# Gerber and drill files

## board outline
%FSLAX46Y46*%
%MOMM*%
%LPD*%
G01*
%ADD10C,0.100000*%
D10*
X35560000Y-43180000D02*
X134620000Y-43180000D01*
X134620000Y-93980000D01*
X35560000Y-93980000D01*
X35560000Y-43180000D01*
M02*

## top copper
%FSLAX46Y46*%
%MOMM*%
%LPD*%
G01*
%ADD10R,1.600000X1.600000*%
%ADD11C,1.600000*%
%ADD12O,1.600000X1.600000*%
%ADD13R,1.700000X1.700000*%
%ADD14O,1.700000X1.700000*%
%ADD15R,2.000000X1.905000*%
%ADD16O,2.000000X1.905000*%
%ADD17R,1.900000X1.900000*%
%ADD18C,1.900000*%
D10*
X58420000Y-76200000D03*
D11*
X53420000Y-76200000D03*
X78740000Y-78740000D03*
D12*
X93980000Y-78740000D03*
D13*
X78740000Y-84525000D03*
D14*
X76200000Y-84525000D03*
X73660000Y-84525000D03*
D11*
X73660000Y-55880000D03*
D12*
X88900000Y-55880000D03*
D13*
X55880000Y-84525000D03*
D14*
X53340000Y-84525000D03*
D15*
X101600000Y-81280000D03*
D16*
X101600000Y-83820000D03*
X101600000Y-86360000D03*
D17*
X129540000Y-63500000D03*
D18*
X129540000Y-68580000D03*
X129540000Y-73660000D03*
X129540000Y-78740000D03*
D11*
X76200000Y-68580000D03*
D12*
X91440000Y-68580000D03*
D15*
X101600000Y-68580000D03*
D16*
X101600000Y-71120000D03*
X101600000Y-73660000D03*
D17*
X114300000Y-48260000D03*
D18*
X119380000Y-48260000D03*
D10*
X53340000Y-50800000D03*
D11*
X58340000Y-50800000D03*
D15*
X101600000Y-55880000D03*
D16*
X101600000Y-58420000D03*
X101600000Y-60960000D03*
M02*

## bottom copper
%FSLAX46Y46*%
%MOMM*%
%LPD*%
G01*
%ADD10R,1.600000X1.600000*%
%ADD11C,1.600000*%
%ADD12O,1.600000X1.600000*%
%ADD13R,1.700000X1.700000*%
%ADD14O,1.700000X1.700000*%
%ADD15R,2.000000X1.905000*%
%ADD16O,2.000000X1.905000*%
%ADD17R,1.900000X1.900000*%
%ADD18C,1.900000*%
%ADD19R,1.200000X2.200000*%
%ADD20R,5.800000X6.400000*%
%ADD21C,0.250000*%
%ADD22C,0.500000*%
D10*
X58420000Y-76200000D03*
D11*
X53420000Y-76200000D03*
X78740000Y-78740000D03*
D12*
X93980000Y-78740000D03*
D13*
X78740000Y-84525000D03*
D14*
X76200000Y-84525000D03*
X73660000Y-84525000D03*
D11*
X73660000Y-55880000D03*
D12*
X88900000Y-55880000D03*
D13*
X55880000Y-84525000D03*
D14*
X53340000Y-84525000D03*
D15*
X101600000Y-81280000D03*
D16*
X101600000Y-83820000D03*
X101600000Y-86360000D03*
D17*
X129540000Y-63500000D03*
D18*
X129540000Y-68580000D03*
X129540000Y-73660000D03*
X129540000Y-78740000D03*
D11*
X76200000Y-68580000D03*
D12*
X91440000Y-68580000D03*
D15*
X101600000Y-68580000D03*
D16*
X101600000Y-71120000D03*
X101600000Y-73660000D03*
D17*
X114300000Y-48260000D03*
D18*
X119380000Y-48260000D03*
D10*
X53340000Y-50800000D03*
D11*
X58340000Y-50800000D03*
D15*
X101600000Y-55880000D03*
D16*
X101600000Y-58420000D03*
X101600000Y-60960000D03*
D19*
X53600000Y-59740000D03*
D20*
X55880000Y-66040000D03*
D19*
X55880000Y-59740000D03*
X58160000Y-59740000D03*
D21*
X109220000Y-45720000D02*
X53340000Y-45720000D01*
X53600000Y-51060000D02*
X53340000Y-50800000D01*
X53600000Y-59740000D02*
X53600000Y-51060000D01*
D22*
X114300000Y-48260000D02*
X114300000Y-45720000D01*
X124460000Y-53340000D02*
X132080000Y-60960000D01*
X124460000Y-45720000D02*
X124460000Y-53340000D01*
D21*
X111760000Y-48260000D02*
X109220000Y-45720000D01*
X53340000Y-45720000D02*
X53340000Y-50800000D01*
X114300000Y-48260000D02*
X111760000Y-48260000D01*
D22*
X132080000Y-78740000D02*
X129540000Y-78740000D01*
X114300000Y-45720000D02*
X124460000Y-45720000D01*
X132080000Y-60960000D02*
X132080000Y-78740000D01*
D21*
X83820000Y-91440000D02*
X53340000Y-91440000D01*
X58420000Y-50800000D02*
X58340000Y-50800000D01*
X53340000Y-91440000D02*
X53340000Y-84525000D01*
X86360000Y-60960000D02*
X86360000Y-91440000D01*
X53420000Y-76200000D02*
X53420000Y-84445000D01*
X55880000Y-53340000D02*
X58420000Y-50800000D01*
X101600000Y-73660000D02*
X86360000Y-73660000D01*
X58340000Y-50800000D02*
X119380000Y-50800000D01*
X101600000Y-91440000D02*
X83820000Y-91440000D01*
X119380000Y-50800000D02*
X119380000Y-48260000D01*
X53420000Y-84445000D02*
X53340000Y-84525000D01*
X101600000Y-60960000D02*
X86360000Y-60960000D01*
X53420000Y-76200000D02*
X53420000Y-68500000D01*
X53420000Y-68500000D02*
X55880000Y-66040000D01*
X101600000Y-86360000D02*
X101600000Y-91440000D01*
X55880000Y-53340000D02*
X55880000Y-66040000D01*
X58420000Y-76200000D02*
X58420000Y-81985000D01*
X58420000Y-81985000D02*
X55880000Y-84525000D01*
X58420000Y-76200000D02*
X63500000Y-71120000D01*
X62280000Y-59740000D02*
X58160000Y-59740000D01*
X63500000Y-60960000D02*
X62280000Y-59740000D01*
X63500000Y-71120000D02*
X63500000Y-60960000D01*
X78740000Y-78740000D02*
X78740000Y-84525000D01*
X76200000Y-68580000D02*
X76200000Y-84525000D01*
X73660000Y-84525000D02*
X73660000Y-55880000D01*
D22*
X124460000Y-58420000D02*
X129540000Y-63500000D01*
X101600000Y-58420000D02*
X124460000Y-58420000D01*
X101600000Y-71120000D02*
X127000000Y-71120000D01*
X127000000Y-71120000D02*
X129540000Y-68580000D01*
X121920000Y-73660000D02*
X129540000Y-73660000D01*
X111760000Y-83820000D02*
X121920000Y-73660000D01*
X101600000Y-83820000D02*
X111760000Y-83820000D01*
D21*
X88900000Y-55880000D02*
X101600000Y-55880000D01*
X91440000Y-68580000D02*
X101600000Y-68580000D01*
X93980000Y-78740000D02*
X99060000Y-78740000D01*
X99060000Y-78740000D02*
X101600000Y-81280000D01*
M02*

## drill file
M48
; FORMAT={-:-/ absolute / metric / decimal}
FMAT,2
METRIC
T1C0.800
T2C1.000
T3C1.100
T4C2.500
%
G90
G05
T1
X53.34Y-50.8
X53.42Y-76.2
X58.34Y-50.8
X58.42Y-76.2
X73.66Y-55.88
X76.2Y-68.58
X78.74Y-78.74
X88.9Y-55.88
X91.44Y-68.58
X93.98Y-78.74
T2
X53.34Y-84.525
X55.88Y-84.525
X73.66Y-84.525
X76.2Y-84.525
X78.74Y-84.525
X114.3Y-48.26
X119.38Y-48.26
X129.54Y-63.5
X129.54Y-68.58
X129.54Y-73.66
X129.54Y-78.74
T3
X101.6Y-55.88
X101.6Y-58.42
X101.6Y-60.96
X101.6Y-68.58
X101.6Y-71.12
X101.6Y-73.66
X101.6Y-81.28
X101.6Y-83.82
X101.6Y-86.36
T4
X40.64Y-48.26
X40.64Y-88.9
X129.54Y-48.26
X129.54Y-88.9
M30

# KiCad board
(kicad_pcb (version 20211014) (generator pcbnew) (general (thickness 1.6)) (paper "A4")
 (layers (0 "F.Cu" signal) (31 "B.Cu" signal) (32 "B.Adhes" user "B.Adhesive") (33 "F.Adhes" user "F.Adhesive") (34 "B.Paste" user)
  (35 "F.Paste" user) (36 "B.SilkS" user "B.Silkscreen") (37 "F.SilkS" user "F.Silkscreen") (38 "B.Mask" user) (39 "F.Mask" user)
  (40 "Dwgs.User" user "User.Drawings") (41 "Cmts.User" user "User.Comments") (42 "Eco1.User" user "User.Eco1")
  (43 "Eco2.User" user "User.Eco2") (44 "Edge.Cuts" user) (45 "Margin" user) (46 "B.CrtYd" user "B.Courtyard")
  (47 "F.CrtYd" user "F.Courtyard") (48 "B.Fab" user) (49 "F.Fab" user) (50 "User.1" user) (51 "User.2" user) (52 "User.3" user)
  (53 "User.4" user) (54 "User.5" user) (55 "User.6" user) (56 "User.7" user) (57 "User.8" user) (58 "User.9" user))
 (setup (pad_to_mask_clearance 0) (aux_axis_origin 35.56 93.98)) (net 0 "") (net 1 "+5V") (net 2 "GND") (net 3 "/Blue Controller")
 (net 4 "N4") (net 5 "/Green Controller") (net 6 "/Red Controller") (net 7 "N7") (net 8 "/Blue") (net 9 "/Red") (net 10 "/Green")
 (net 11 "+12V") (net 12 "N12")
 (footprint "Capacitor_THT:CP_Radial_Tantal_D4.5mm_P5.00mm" (layer "F.Cu") (at 58.42 76.2 180)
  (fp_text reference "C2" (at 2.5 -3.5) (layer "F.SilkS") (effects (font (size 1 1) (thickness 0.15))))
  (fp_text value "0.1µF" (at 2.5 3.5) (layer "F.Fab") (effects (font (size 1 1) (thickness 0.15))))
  (pad "1" thru_hole rect (at 0 0 180) (size 1.6 1.6) (drill 0.8) (layers *.Cu *.Mask) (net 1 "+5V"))
  (pad "2" thru_hole circle (at 5 0 180) (size 1.6 1.6) (drill 0.8) (layers *.Cu *.Mask) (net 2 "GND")))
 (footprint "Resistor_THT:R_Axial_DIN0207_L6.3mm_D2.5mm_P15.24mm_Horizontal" (layer "F.Cu") (at 78.74 78.74)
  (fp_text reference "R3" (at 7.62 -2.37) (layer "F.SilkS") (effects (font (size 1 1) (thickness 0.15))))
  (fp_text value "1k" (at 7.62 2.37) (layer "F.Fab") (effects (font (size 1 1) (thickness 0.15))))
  (pad "1" thru_hole circle (at 0 0) (size 1.6 1.6) (drill 0.8) (layers *.Cu *.Mask) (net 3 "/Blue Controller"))
  (pad "2" thru_hole oval (at 15.24 0) (size 1.6 1.6) (drill 0.8) (layers *.Cu *.Mask) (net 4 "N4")))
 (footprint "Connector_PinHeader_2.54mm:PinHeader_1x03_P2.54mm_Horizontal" (layer "F.Cu") (at 78.74 84.525 -90)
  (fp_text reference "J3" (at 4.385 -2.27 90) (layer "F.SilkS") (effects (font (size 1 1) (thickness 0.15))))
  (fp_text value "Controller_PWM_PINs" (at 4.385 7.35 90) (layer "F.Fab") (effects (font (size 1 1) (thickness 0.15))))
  (pad "1" thru_hole rect (at 0 0 270) (size 1.7 1.7) (drill 1) (layers *.Cu *.Mask) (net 3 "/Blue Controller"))
  (pad "2" thru_hole oval (at 0 2.54 270) (size 1.7 1.7) (drill 1) (layers *.Cu *.Mask) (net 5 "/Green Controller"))
  (pad "3" thru_hole oval (at 0 5.08 270) (size 1.7 1.7) (drill 1) (layers *.Cu *.Mask) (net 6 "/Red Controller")))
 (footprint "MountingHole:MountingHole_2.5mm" (layer "F.Cu") (at 129.54 48.26)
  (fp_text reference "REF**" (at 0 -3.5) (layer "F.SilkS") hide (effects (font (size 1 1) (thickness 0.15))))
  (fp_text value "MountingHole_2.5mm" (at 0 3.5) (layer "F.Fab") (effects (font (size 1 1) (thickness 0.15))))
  (pad "" np_thru_hole circle (at 0 0) (size 2.5 2.5) (drill 2.5) (layers *.Cu *.Mask)))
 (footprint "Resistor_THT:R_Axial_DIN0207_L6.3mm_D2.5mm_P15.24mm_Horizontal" (layer "F.Cu") (at 73.66 55.88)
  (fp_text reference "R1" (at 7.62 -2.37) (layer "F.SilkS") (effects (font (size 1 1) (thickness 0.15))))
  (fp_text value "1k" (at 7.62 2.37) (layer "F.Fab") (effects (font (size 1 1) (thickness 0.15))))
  (pad "1" thru_hole circle (at 0 0) (size 1.6 1.6) (drill 0.8) (layers *.Cu *.Mask) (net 6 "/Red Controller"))
  (pad "2" thru_hole oval (at 15.24 0) (size 1.6 1.6) (drill 0.8) (layers *.Cu *.Mask) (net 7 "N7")))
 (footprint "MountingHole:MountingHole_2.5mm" (layer "F.Cu") (at 40.64 48.26)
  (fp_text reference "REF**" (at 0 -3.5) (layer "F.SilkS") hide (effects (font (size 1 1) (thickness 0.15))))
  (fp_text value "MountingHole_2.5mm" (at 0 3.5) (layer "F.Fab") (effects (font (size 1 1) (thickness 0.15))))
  (pad "" np_thru_hole circle (at 0 0) (size 2.5 2.5) (drill 2.5) (layers *.Mask)))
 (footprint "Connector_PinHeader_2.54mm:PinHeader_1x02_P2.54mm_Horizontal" (layer "F.Cu") (at 55.88 84.525 -90)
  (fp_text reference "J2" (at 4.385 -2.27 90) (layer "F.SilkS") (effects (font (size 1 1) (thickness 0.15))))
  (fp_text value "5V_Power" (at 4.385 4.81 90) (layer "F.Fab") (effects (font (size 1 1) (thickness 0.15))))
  (pad "1" thru_hole rect (at 0 0 270) (size 1.7 1.7) (drill 1) (layers *.Cu *.Mask) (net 1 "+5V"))
  (pad "2" thru_hole oval (at 0 2.54 270) (size 1.7 1.7) (drill 1) (layers *.Cu *.Mask) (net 2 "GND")))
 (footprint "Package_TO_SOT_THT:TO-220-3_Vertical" (layer "F.Cu") (at 101.6 81.28 -90)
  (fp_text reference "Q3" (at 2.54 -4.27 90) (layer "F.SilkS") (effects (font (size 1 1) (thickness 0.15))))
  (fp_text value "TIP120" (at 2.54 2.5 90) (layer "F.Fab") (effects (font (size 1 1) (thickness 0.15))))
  (pad "1" thru_hole rect (at 0 0 270) (size 1.905 2) (drill 1.1) (layers *.Cu *.Mask) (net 4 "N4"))
  (pad "2" thru_hole oval (at 2.54 0 270) (size 1.905 2) (drill 1.1) (layers *.Cu *.Mask) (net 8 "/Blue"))
  (pad "3" thru_hole oval (at 5.08 0 270) (size 1.905 2) (drill 1.1) (layers *.Cu *.Mask) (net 2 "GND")))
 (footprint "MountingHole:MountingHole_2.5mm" (layer "F.Cu") (at 129.54 88.9)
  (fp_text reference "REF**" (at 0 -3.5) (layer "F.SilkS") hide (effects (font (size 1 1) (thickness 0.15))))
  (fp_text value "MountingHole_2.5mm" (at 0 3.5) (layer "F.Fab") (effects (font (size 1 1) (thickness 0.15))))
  (pad "" np_thru_hole circle (at 0 0) (size 2.5 2.5) (drill 2.5) (layers *.Cu *.Mask)))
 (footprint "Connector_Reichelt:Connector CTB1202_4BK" (layer "F.Cu") (at 129.54 63.5 -90)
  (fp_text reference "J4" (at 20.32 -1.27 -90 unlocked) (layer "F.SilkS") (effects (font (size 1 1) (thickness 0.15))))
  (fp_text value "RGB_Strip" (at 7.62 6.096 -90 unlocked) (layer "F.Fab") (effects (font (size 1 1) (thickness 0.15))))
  (pad "1" thru_hole rect (at 0 0 270) (size 1.9 1.9) (drill 1) (layers *.Cu *.Mask) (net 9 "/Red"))
  (pad "2" thru_hole circle (at 5.08 0 270) (size 1.9 1.9) (drill 1) (layers *.Cu *.Mask) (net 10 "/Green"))
  (pad "3" thru_hole circle (at 10.16 0 270) (size 1.9 1.9) (drill 1) (layers *.Cu *.Mask) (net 8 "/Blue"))
  (pad "4" thru_hole circle (at 15.24 0 270) (size 1.9 1.9) (drill 1) (layers *.Cu *.Mask) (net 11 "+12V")))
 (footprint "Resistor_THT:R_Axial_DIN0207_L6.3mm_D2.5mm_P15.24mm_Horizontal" (layer "F.Cu") (at 76.2 68.58)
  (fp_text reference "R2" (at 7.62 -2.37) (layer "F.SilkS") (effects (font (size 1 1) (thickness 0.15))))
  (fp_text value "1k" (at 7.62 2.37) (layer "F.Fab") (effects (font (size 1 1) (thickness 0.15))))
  (pad "1" thru_hole circle (at 0 0) (size 1.6 1.6) (drill 0.8) (layers *.Cu *.Mask) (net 5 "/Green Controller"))
  (pad "2" thru_hole oval (at 15.24 0) (size 1.6 1.6) (drill 0.8) (layers *.Cu *.Mask) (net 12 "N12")))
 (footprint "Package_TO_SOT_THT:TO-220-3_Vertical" (layer "F.Cu") (at 101.6 68.58 -90)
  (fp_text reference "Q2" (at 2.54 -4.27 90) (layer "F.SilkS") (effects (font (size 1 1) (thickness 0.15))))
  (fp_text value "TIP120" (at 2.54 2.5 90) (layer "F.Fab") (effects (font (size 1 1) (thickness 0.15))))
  (pad "1" thru_hole rect (at 0 0 270) (size 1.905 2) (drill 1.1) (layers *.Cu *.Mask) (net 12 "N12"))
  (pad "2" thru_hole oval (at 2.54 0 270) (size 1.905 2) (drill 1.1) (layers *.Cu *.Mask) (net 10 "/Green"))
  (pad "3" thru_hole oval (at 5.08 0 270) (size 1.905 2) (drill 1.1) (layers *.Cu *.Mask) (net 2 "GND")))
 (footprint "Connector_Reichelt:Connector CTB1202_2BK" (layer "F.Cu") (at 114.3 48.26)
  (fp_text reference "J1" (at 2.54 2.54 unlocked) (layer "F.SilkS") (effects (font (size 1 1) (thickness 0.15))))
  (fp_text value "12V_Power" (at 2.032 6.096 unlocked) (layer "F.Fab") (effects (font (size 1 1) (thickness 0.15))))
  (pad "1" thru_hole rect (at 0 0) (size 1.9 1.9) (drill 1) (layers *.Cu *.Mask) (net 11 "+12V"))
  (pad "2" thru_hole circle (at 5.08 0) (size 1.9 1.9) (drill 1) (layers *.Cu *.Mask) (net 2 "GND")))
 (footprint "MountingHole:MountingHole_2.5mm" (layer "F.Cu") (at 40.64 88.9)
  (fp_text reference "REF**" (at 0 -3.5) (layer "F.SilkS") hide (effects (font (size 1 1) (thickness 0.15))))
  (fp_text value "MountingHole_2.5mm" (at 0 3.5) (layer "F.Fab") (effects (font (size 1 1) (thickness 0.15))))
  (pad "" np_thru_hole circle (at 0 0) (size 2.5 2.5) (drill 2.5) (layers *.Cu *.Mask)))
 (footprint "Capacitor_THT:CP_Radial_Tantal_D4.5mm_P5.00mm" (layer "F.Cu") (at 53.34 50.8)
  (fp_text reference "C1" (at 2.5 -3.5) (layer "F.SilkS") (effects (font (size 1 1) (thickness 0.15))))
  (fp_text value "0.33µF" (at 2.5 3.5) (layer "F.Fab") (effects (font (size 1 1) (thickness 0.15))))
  (pad "1" thru_hole rect (at 0 0) (size 1.6 1.6) (drill 0.8) (layers *.Cu *.Mask) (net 11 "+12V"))
  (pad "2" thru_hole circle (at 5 0) (size 1.6 1.6) (drill 0.8) (layers *.Cu *.Mask) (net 2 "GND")))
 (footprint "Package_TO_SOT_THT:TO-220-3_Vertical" (layer "F.Cu") (at 101.6 55.88 -90)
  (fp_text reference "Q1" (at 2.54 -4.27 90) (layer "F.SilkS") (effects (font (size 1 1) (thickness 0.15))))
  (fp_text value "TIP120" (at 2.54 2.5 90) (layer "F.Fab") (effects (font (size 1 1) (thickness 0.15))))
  (pad "1" thru_hole rect (at 0 0 270) (size 1.905 2) (drill 1.1) (layers *.Cu *.Mask) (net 7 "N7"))
  (pad "2" thru_hole oval (at 2.54 0 270) (size 1.905 2) (drill 1.1) (layers *.Cu *.Mask) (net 9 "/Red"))
  (pad "3" thru_hole oval (at 5.08 0 270) (size 1.905 2) (drill 1.1) (layers *.Cu *.Mask) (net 2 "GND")))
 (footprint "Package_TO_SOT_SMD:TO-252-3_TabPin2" (layer "B.Cu") (at 55.88 63.94 -90)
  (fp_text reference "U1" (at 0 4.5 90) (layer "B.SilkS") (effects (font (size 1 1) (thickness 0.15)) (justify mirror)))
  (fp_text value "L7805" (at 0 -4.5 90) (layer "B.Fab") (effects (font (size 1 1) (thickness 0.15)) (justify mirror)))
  (pad "" smd rect (at 0.425 1.525 270) (size 3.05 2.75) (layers "B.Paste"))
  (pad "" smd rect (at 0.425 -1.525 270) (size 3.05 2.75) (layers "B.Paste"))
  (pad "" smd rect (at 3.775 -1.525 270) (size 3.05 2.75) (layers "B.Paste"))
  (pad "" smd rect (at 3.775 1.525 270) (size 3.05 2.75) (layers "B.Paste"))
  (pad "1" smd rect (at -4.2 2.28 270) (size 2.2 1.2) (layers "B.Cu" "B.Paste" "B.Mask") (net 11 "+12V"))
  (pad "2" smd rect (at 2.1 0 270) (size 6.4 5.8) (layers "B.Cu" "B.Mask") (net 2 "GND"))
  (pad "2" smd rect (at -4.2 0 270) (size 2.2 1.2) (layers "B.Cu" "B.Paste" "B.Mask") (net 2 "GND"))
  (pad "3" smd rect (at -4.2 -2.28 270) (size 2.2 1.2) (layers "B.Cu" "B.Paste" "B.Mask") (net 1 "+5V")))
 (gr_rect (start 35.56 43.18) (end 134.62 93.98) (layer "Edge.Cuts") (width 0.1) (fill none))
 (segment (start 109.22 45.72) (end 53.34 45.72) (width 0.25) (layer "B.Cu") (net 11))
 (segment (start 53.6 51.06) (end 53.34 50.8) (width 0.25) (layer "B.Cu") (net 11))
 (segment (start 53.6 59.74) (end 53.6 51.06) (width 0.25) (layer "B.Cu") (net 11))
 (segment (start 114.3 48.26) (end 114.3 45.72) (width 0.5) (layer "B.Cu") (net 11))
 (segment (start 124.46 53.34) (end 132.08 60.96) (width 0.5) (layer "B.Cu") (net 11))
 (segment (start 124.46 45.72) (end 124.46 53.34) (width 0.5) (layer "B.Cu") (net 11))
 (segment (start 111.76 48.26) (end 109.22 45.72) (width 0.25) (layer "B.Cu") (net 11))
 (segment (start 53.34 45.72) (end 53.34 50.8) (width 0.25) (layer "B.Cu") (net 11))
 (segment (start 114.3 48.26) (end 111.76 48.26) (width 0.25) (layer "B.Cu") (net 11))
 (segment (start 132.08 78.74) (end 129.54 78.74) (width 0.5) (layer "B.Cu") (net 11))
 (segment (start 114.3 45.72) (end 124.46 45.72) (width 0.5) (layer "B.Cu") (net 11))
 (segment (start 132.08 60.96) (end 132.08 78.74) (width 0.5) (layer "B.Cu") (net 11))
 (segment (start 83.82 91.44) (end 53.34 91.44) (width 0.25) (layer "B.Cu") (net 2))
 (segment (start 58.42 50.8) (end 58.34 50.8) (width 0.25) (layer "B.Cu") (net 2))
 (segment (start 53.34 91.44) (end 53.34 84.525) (width 0.25) (layer "B.Cu") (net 2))
 (segment (start 86.36 60.96) (end 86.36 91.44) (width 0.25) (layer "B.Cu") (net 2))
 (segment (start 53.42 76.2) (end 53.42 84.445) (width 0.25) (layer "B.Cu") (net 2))
 (segment (start 55.88 53.34) (end 58.42 50.8) (width 0.25) (layer "B.Cu") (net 2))
 (segment (start 101.6 73.66) (end 86.36 73.66) (width 0.25) (layer "B.Cu") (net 2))
 (segment (start 58.34 50.8) (end 119.38 50.8) (width 0.25) (layer "B.Cu") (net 2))
 (segment (start 101.6 91.44) (end 83.82 91.44) (width 0.25) (layer "B.Cu") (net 2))
 (segment (start 119.38 50.8) (end 119.38 48.26) (width 0.25) (layer "B.Cu") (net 2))
 (segment (start 53.42 84.445) (end 53.34 84.525) (width 0.25) (layer "B.Cu") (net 2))
 (segment (start 101.6 60.96) (end 86.36 60.96) (width 0.25) (layer "B.Cu") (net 2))
 (segment (start 53.42 76.2) (end 53.42 68.5) (width 0.25) (layer "B.Cu") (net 2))
 (segment (start 53.42 68.5) (end 55.88 66.04) (width 0.25) (layer "B.Cu") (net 2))
 (segment (start 101.6 86.36) (end 101.6 91.44) (width 0.25) (layer "B.Cu") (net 2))
 (segment (start 55.88 53.34) (end 55.88 66.04) (width 0.25) (layer "B.Cu") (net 2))
 (segment (start 58.42 76.2) (end 58.42 81.985) (width 0.25) (layer "B.Cu") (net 1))
 (segment (start 58.42 81.985) (end 55.88 84.525) (width 0.25) (layer "B.Cu") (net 1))
 (segment (start 58.42 76.2) (end 63.5 71.12) (width 0.25) (layer "B.Cu") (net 1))
 (segment (start 62.28 59.74) (end 58.16 59.74) (width 0.25) (layer "B.Cu") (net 1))
 (segment (start 63.5 60.96) (end 62.28 59.74) (width 0.25) (layer "B.Cu") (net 1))
 (segment (start 63.5 71.12) (end 63.5 60.96) (width 0.25) (layer "B.Cu") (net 1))
 (segment (start 78.74 78.74) (end 78.74 84.525) (width 0.25) (layer "B.Cu") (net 3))
 (segment (start 76.2 68.58) (end 76.2 84.525) (width 0.25) (layer "B.Cu") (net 5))
 (segment (start 73.66 84.525) (end 73.66 55.88) (width 0.25) (layer "B.Cu") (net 6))
 (segment (start 124.46 58.42) (end 129.54 63.5) (width 0.5) (layer "B.Cu") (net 9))
 (segment (start 101.6 58.42) (end 124.46 58.42) (width 0.5) (layer "B.Cu") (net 9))
 (segment (start 101.6 71.12) (end 127 71.12) (width 0.5) (layer "B.Cu") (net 10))
 (segment (start 127 71.12) (end 129.54 68.58) (width 0.5) (layer "B.Cu") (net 10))
 (segment (start 121.92 73.66) (end 129.54 73.66) (width 0.5) (layer "B.Cu") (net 8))
 (segment (start 111.76 83.82) (end 121.92 73.66) (width 0.5) (layer "B.Cu") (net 8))
 (segment (start 101.6 83.82) (end 111.76 83.82) (width 0.5) (layer "B.Cu") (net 8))
 (segment (start 88.9 55.88) (end 101.6 55.88) (width 0.25) (layer "B.Cu") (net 7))
 (segment (start 91.44 68.58) (end 101.6 68.58) (width 0.25) (layer "B.Cu") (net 12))
 (segment (start 93.98 78.74) (end 99.06 78.74) (width 0.25) (layer "B.Cu") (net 4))
 (segment (start 99.06 78.74) (end 101.6 81.28) (width 0.25) (layer "B.Cu") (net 4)))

